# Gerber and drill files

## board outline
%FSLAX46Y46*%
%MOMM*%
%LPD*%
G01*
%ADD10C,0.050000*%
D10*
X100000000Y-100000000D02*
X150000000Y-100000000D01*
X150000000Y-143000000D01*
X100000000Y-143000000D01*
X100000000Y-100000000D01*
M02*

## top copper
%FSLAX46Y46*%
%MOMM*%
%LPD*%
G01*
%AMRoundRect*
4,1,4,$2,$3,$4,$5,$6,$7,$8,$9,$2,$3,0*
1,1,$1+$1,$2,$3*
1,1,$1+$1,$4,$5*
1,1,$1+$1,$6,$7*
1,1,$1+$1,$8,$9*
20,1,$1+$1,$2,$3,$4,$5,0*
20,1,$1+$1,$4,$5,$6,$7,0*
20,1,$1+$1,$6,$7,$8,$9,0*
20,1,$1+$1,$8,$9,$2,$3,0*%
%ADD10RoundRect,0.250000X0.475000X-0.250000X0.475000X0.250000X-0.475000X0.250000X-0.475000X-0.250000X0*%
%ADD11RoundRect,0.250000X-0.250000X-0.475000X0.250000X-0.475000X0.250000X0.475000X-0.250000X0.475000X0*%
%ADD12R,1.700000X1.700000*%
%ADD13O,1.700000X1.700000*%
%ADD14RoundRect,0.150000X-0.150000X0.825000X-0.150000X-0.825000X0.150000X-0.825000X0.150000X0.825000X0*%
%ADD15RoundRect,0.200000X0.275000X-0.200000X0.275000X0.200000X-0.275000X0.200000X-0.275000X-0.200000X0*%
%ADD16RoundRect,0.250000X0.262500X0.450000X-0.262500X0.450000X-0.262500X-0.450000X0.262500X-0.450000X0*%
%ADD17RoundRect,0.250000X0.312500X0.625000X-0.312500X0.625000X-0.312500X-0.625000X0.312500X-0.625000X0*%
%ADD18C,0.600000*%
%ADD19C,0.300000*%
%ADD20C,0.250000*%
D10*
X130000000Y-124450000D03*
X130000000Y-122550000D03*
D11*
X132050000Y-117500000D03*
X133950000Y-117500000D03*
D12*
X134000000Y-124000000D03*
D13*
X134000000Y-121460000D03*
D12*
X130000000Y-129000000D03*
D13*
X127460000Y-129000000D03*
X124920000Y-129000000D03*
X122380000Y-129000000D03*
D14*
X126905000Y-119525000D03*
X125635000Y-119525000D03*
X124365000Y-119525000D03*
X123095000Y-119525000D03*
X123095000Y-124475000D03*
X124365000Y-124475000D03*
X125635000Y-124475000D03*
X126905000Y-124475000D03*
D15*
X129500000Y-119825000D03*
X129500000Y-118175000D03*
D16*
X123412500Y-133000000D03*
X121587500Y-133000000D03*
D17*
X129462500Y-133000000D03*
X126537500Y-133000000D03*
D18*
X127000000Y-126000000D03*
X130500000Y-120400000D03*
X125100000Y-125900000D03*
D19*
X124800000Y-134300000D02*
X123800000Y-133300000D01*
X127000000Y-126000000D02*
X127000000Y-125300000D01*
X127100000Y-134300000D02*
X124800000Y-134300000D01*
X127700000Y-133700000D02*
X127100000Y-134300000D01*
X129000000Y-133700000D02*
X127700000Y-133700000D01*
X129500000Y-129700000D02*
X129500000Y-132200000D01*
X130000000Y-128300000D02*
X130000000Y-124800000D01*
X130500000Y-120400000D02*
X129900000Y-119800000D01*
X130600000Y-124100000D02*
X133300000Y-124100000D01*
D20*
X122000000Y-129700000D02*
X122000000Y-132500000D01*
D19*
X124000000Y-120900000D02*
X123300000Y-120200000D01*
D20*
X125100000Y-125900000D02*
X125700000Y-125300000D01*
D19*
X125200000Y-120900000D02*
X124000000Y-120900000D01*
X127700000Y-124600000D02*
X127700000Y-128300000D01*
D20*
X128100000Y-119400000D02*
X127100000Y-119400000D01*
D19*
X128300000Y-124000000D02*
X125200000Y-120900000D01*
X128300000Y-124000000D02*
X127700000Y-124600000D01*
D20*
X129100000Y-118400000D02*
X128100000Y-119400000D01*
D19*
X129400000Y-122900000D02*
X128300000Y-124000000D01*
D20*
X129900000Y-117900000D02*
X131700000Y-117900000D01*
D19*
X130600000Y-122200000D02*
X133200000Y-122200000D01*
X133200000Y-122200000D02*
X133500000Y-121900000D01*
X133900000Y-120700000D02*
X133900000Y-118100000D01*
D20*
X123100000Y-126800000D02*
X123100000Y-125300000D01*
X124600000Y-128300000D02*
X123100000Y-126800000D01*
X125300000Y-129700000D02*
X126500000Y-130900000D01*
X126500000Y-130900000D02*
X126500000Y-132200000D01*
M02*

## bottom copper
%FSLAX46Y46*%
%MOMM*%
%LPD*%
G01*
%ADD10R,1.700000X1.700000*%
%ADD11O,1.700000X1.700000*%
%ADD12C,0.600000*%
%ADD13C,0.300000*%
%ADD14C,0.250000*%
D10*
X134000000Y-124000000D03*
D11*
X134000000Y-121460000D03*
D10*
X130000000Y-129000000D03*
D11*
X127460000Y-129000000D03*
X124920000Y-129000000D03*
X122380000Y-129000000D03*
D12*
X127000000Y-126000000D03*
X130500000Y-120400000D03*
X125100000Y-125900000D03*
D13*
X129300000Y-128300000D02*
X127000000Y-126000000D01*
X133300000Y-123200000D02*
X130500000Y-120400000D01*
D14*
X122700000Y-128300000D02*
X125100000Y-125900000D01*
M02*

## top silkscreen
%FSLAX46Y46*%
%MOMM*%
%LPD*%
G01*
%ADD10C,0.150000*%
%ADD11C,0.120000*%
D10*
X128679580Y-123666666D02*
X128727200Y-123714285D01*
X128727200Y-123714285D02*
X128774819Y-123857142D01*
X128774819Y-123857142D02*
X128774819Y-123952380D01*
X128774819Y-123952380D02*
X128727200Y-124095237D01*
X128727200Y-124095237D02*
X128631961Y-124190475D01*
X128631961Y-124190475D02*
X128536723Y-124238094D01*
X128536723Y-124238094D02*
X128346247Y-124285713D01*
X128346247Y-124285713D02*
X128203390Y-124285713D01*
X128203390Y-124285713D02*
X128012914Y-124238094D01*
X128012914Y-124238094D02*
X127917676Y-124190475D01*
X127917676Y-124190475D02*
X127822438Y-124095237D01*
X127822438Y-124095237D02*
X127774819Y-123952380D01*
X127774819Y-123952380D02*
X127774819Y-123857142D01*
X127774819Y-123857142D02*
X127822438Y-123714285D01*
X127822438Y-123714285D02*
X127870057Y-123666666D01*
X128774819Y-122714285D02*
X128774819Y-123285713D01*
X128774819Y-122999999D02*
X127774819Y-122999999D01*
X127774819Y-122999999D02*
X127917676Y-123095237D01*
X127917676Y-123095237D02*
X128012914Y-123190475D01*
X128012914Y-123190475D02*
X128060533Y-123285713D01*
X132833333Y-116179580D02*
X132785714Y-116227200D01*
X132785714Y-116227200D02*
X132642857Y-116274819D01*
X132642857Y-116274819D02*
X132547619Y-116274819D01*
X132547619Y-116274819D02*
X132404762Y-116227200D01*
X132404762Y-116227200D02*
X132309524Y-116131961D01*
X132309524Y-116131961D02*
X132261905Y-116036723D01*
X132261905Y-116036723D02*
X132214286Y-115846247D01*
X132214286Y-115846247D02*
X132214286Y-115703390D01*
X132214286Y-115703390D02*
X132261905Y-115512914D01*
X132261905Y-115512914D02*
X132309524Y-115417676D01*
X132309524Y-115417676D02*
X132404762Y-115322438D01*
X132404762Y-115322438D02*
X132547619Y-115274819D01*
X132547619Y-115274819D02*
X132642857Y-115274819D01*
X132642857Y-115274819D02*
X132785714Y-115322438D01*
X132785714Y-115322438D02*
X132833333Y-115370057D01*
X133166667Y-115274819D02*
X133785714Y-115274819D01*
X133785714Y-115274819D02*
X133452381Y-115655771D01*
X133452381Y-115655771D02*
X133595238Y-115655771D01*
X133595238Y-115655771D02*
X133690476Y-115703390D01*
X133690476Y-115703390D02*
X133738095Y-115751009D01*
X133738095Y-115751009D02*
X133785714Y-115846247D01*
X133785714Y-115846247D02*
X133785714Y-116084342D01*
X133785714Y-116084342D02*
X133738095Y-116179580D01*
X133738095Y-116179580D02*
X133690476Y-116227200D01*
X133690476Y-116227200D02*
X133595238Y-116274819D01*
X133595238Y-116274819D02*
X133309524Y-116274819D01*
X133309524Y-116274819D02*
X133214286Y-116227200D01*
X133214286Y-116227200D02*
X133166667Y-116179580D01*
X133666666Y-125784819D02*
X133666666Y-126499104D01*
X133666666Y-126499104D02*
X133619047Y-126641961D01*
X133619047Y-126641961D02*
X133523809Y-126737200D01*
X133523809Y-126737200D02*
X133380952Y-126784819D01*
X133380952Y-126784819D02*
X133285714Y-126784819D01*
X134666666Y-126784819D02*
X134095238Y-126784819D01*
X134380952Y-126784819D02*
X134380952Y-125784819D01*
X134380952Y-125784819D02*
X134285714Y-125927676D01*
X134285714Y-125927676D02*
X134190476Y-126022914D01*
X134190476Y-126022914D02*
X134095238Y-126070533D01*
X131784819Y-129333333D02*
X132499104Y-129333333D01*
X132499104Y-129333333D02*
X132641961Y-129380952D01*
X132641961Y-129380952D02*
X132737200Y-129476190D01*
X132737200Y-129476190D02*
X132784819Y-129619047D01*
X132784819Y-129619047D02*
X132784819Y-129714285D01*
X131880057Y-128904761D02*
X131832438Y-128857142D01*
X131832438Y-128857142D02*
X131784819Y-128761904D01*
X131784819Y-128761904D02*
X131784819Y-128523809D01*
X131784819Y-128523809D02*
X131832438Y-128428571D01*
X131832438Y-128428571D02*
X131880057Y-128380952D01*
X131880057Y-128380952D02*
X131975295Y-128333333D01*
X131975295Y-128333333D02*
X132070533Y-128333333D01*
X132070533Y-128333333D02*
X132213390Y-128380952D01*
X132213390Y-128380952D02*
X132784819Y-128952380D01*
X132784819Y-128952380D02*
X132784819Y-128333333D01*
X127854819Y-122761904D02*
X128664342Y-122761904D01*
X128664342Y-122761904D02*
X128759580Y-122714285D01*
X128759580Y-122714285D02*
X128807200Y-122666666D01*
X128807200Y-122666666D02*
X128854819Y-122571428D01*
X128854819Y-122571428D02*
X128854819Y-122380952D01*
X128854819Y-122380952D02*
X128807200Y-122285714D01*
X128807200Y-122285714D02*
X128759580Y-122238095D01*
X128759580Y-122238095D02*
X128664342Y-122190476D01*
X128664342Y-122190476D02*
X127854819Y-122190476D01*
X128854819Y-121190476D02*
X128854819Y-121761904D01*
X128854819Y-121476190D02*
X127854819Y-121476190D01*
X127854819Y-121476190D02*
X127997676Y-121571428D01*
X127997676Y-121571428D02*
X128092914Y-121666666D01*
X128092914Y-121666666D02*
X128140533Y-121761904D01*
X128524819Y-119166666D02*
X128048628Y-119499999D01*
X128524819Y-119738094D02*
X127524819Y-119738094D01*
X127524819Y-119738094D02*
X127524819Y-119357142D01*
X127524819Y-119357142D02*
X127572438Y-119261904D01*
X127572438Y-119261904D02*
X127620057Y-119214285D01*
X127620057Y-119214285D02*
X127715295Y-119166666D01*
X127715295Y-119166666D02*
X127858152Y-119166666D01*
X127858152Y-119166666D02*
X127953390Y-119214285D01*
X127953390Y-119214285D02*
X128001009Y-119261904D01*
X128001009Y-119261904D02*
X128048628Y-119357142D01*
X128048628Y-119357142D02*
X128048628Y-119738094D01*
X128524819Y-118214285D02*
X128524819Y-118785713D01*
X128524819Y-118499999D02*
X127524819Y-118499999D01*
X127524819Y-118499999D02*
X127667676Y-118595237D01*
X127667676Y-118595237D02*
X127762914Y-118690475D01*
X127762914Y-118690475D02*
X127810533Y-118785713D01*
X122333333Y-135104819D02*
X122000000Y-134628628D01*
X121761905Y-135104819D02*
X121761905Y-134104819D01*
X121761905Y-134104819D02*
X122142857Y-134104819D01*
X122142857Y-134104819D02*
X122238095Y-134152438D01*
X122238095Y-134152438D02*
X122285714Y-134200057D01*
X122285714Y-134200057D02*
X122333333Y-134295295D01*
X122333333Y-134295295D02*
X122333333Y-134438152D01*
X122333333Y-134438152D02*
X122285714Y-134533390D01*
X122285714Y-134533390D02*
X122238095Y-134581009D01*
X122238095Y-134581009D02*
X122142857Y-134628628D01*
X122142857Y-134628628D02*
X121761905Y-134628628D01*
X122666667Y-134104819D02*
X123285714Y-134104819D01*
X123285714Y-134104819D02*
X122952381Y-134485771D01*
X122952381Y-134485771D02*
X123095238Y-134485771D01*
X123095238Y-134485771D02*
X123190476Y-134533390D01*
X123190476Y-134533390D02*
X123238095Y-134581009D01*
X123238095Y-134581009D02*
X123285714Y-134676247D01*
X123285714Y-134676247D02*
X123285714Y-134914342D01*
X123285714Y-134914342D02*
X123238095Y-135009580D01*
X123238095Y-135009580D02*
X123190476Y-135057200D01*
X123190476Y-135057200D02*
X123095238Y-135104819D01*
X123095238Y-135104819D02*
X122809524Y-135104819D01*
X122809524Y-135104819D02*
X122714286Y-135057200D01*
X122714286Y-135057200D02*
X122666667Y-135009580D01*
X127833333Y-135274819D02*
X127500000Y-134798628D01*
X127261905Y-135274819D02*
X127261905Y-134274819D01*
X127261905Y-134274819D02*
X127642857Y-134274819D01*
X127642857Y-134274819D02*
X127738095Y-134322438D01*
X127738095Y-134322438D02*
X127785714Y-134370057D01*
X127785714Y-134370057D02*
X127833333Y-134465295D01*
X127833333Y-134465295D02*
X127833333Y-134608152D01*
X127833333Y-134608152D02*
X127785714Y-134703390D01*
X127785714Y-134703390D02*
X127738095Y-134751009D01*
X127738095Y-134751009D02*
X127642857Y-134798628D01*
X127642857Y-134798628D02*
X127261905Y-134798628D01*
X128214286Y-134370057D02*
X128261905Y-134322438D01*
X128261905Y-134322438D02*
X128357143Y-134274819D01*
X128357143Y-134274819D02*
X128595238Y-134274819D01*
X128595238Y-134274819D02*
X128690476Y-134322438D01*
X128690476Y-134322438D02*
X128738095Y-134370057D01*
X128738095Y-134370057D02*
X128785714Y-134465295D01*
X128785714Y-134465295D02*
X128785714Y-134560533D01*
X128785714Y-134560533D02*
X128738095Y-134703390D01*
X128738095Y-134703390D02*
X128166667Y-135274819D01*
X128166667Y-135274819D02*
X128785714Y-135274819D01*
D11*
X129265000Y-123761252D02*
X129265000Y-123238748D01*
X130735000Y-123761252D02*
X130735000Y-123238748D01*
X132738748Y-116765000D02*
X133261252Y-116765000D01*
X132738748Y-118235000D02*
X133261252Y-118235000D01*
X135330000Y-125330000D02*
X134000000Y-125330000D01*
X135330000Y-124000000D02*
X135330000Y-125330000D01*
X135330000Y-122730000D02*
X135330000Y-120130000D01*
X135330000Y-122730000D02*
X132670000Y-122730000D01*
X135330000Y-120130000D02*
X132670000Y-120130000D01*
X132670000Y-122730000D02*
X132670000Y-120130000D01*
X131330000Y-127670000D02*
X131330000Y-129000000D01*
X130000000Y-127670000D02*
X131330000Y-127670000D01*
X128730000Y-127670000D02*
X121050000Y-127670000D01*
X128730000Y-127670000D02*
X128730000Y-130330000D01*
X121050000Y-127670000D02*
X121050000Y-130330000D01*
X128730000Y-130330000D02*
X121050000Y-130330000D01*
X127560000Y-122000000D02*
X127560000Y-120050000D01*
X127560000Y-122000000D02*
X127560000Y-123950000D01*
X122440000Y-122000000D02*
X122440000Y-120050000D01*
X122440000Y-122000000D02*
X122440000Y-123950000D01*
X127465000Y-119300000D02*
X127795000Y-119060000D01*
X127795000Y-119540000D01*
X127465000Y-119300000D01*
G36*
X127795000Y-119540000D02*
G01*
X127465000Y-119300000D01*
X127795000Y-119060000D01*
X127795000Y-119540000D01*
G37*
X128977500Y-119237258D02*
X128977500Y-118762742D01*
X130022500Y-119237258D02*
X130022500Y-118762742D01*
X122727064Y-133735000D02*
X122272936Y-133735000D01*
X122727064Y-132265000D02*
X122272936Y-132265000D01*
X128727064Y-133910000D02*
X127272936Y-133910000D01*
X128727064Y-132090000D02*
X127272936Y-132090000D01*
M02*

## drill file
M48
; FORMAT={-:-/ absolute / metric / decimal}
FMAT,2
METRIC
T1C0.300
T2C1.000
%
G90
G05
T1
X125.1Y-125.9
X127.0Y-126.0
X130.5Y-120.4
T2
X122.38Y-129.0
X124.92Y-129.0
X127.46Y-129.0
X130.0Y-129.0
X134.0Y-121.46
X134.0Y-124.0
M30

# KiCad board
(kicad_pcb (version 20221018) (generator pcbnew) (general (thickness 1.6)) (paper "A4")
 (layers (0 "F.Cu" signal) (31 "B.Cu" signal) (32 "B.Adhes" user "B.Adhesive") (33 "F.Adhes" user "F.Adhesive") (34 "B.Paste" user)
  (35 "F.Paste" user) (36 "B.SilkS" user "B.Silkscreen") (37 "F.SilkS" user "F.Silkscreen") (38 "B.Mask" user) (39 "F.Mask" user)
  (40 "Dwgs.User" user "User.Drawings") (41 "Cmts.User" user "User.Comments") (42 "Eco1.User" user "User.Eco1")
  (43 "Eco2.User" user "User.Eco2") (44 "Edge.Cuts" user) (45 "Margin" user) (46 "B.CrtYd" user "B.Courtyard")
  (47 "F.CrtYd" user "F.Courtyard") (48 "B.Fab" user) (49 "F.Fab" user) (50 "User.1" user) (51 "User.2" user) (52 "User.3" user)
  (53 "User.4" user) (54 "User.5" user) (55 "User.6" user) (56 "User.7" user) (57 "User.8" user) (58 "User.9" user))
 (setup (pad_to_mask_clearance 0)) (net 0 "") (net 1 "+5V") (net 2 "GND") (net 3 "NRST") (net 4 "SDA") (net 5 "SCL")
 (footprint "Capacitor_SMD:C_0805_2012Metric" (layer "F.Cu") (at 130 123.5 90)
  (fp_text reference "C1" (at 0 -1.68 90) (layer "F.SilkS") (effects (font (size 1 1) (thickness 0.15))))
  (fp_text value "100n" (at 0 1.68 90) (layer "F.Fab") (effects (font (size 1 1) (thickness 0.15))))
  (fp_line (start -0.261252 -0.735) (end 0.261252 -0.735) (stroke (width 0.12) (type solid)) (layer "F.SilkS"))
  (fp_line (start -0.261252 0.735) (end 0.261252 0.735) (stroke (width 0.12) (type solid)) (layer "F.SilkS"))
  (pad "1" smd roundrect (at -0.95 0 90) (size 1 1.45) (layers "F.Cu" "F.Paste" "F.Mask") (roundrect_rratio 0.25) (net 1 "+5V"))
  (pad "2" smd roundrect (at 0.95 0 90) (size 1 1.45) (layers "F.Cu" "F.Paste" "F.Mask") (roundrect_rratio 0.25) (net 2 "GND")))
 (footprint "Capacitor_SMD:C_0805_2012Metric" (layer "F.Cu") (at 133 117.5)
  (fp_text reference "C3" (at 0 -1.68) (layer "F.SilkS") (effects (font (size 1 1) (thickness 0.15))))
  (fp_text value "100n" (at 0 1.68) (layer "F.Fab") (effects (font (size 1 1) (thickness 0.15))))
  (fp_line (start -0.261252 -0.735) (end 0.261252 -0.735) (stroke (width 0.12) (type solid)) (layer "F.SilkS"))
  (fp_line (start -0.261252 0.735) (end 0.261252 0.735) (stroke (width 0.12) (type solid)) (layer "F.SilkS"))
  (pad "1" smd roundrect (at -0.95 0) (size 1 1.45) (layers "F.Cu" "F.Paste" "F.Mask") (roundrect_rratio 0.25) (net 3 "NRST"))
  (pad "2" smd roundrect (at 0.95 0) (size 1 1.45) (layers "F.Cu" "F.Paste" "F.Mask") (roundrect_rratio 0.25) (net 2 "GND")))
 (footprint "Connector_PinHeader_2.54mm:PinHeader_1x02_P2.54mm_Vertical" (layer "F.Cu") (at 134 124 180)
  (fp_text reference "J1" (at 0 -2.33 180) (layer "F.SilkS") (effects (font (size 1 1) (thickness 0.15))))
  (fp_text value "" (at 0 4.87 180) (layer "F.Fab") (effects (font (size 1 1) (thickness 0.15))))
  (fp_line (start -1.33 -1.33) (end 0 -1.33) (stroke (width 0.12) (type solid)) (layer "F.SilkS"))
  (fp_line (start -1.33 0) (end -1.33 -1.33) (stroke (width 0.12) (type solid)) (layer "F.SilkS"))
  (fp_line (start -1.33 1.27) (end -1.33 3.87) (stroke (width 0.12) (type solid)) (layer "F.SilkS"))
  (fp_line (start -1.33 1.27) (end 1.33 1.27) (stroke (width 0.12) (type solid)) (layer "F.SilkS"))
  (fp_line (start -1.33 3.87) (end 1.33 3.87) (stroke (width 0.12) (type solid)) (layer "F.SilkS"))
  (fp_line (start 1.33 1.27) (end 1.33 3.87) (stroke (width 0.12) (type solid)) (layer "F.SilkS"))
  (pad "1" thru_hole rect (at 0 0 180) (size 1.7 1.7) (drill 1) (layers "*.Cu" "*.Mask") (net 1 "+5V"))
  (pad "2" thru_hole oval (at 0 2.54 180) (size 1.7 1.7) (drill 1) (layers "*.Cu" "*.Mask") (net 2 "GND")))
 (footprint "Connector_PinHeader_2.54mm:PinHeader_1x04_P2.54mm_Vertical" (layer "F.Cu") (at 130 129 -90)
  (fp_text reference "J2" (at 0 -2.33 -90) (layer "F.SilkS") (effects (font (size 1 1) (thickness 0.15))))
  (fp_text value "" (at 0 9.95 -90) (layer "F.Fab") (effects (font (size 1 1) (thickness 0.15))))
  (fp_line (start -1.33 -1.33) (end 0 -1.33) (stroke (width 0.12) (type solid)) (layer "F.SilkS"))
  (fp_line (start -1.33 0) (end -1.33 -1.33) (stroke (width 0.12) (type solid)) (layer "F.SilkS"))
  (fp_line (start -1.33 1.27) (end -1.33 8.95) (stroke (width 0.12) (type solid)) (layer "F.SilkS"))
  (fp_line (start -1.33 1.27) (end 1.33 1.27) (stroke (width 0.12) (type solid)) (layer "F.SilkS"))
  (fp_line (start -1.33 8.95) (end 1.33 8.95) (stroke (width 0.12) (type solid)) (layer "F.SilkS"))
  (fp_line (start 1.33 1.27) (end 1.33 8.95) (stroke (width 0.12) (type solid)) (layer "F.SilkS"))
  (pad "1" thru_hole rect (at 0 0 270) (size 1.7 1.7) (drill 1) (layers "*.Cu" "*.Mask") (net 1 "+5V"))
  (pad "2" thru_hole oval (at 0 2.54 270) (size 1.7 1.7) (drill 1) (layers "*.Cu" "*.Mask") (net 2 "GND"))
  (pad "3" thru_hole oval (at 0 5.08 270) (size 1.7 1.7) (drill 1) (layers "*.Cu" "*.Mask") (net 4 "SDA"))
  (pad "4" thru_hole oval (at 0 7.62 270) (size 1.7 1.7) (drill 1) (layers "*.Cu" "*.Mask") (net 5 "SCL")))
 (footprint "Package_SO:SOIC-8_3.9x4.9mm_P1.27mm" (layer "F.Cu") (at 125 122 -90)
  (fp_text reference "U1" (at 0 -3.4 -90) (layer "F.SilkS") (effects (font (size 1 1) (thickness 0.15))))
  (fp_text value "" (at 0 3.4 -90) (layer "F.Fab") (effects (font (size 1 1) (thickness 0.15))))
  (fp_line (start 0 -2.56) (end -1.95 -2.56) (stroke (width 0.12) (type solid)) (layer "F.SilkS"))
  (fp_line (start 0 -2.56) (end 1.95 -2.56) (stroke (width 0.12) (type solid)) (layer "F.SilkS"))
  (fp_line (start 0 2.56) (end -1.95 2.56) (stroke (width 0.12) (type solid)) (layer "F.SilkS"))
  (fp_line (start 0 2.56) (end 1.95 2.56) (stroke (width 0.12) (type solid)) (layer "F.SilkS"))
  (fp_poly
   (pts (xy -2.7 -2.465) (xy -2.94 -2.795) (xy -2.46 -2.795) (xy -2.7 -2.465)) (stroke (width 0.12) (type solid)) (fill solid)
   (layer "F.SilkS"))
  (pad "1" smd roundrect (at -2.475 -1.905 270) (size 1.95 0.6) (layers "F.Cu" "F.Paste" "F.Mask") (roundrect_rratio 0.25) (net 3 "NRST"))
  (pad "2" smd roundrect (at -2.475 -0.635 270) (size 1.95 0.6) (layers "F.Cu" "F.Paste" "F.Mask") (roundrect_rratio 0.25))
  (pad "3" smd roundrect (at -2.475 0.635 270) (size 1.95 0.6) (layers "F.Cu" "F.Paste" "F.Mask") (roundrect_rratio 0.25))
  (pad "4" smd roundrect (at -2.475 1.905 270) (size 1.95 0.6) (layers "F.Cu" "F.Paste" "F.Mask") (roundrect_rratio 0.25) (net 2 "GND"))
  (pad "5" smd roundrect (at 2.475 1.905 270) (size 1.95 0.6) (layers "F.Cu" "F.Paste" "F.Mask") (roundrect_rratio 0.25) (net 4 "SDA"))
  (pad "6" smd roundrect (at 2.475 0.635 270) (size 1.95 0.6) (layers "F.Cu" "F.Paste" "F.Mask") (roundrect_rratio 0.25))
  (pad "7" smd roundrect (at 2.475 -0.635 270) (size 1.95 0.6) (layers "F.Cu" "F.Paste" "F.Mask") (roundrect_rratio 0.25) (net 5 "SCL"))
  (pad "8" smd roundrect (at 2.475 -1.905 270) (size 1.95 0.6) (layers "F.Cu" "F.Paste" "F.Mask") (roundrect_rratio 0.25) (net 1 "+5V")))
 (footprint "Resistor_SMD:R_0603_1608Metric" (layer "F.Cu") (at 129.5 119 90)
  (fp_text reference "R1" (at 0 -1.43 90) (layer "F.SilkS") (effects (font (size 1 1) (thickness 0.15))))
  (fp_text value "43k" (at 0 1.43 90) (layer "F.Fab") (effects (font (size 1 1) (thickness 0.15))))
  (fp_line (start -0.237258 -0.5225) (end 0.237258 -0.5225) (stroke (width 0.12) (type solid)) (layer "F.SilkS"))
  (fp_line (start -0.237258 0.5225) (end 0.237258 0.5225) (stroke (width 0.12) (type solid)) (layer "F.SilkS"))
  (pad "1" smd roundrect (at -0.825 0 90) (size 0.8 0.95) (layers "F.Cu" "F.Paste" "F.Mask") (roundrect_rratio 0.25) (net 1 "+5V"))
  (pad "2" smd roundrect (at 0.825 0 90) (size 0.8 0.95) (layers "F.Cu" "F.Paste" "F.Mask") (roundrect_rratio 0.25) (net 3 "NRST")))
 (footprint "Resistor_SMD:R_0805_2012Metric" (layer "F.Cu") (at 122.5 133 180)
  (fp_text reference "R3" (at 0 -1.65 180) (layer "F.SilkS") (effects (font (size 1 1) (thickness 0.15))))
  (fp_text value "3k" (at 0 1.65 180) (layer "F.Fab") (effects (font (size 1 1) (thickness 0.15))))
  (fp_line (start -0.227064 -0.735) (end 0.227064 -0.735) (stroke (width 0.12) (type solid)) (layer "F.SilkS"))
  (fp_line (start -0.227064 0.735) (end 0.227064 0.735) (stroke (width 0.12) (type solid)) (layer "F.SilkS"))
  (pad "1" smd roundrect (at -0.9125 0 180) (size 1.025 1.4) (layers "F.Cu" "F.Paste" "F.Mask") (roundrect_rratio 0.243902) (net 1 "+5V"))
  (pad "2" smd roundrect (at 0.9125 0 180) (size 1.025 1.4) (layers "F.Cu" "F.Paste" "F.Mask") (roundrect_rratio 0.243902) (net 5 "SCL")))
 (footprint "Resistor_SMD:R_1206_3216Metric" (layer "F.Cu") (at 128 133 180)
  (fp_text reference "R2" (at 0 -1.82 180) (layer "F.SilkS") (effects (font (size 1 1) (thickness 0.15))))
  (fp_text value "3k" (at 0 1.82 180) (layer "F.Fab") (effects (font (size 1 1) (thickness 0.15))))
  (fp_line (start -0.727064 -0.91) (end 0.727064 -0.91) (stroke (width 0.12) (type solid)) (layer "F.SilkS"))
  (fp_line (start -0.727064 0.91) (end 0.727064 0.91) (stroke (width 0.12) (type solid)) (layer "F.SilkS"))
  (pad "1" smd roundrect (at -1.4625 0 180) (size 1.125 1.75) (layers "F.Cu" "F.Paste" "F.Mask") (roundrect_rratio 0.222222) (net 1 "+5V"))
  (pad "2" smd roundrect (at 1.4625 0 180) (size 1.125 1.75) (layers "F.Cu" "F.Paste" "F.Mask") (roundrect_rratio 0.222222) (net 4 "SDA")))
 (gr_rect (start 100 100) (end 150 143) (stroke (width 0.05) (type default)) (fill none) (layer "Edge.Cuts"))
 (segment (start 124.8 134.3) (end 123.8 133.3) (width 0.3) (layer "F.Cu") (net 1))
 (segment (start 127 126) (end 127 125.3) (width 0.3) (layer "F.Cu") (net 1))
 (segment (start 127.1 134.3) (end 124.8 134.3) (width 0.3) (layer "F.Cu") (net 1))
 (segment (start 127.7 133.7) (end 127.1 134.3) (width 0.3) (layer "F.Cu") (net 1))
 (segment (start 129 133.7) (end 127.7 133.7) (width 0.3) (layer "F.Cu") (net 1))
 (segment (start 129.5 129.7) (end 129.5 132.2) (width 0.3) (layer "F.Cu") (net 1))
 (segment (start 130 128.3) (end 130 124.8) (width 0.3) (layer "F.Cu") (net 1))
 (segment (start 130.5 120.4) (end 129.9 119.8) (width 0.3) (layer "F.Cu") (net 1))
 (segment (start 130.6 124.1) (end 133.3 124.1) (width 0.3) (layer "F.Cu") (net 1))
 (via (at 127 126) (size 0.6) (drill 0.3) (layers "F.Cu" "B.Cu") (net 1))
 (via (at 130.5 120.4) (size 0.6) (drill 0.3) (layers "F.Cu" "B.Cu") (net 1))
 (segment (start 122 129.7) (end 122 132.5) (width 0.25) (layer "F.Cu") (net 5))
 (segment (start 124 120.9) (end 123.3 120.2) (width 0.3) (layer "F.Cu") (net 2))
 (segment (start 125.1 125.9) (end 125.7 125.3) (width 0.25) (layer "F.Cu") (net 5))
 (segment (start 125.2 120.9) (end 124 120.9) (width 0.3) (layer "F.Cu") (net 2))
 (segment (start 127.7 124.6) (end 127.7 128.3) (width 0.3) (layer "F.Cu") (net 2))
 (segment (start 128.1 119.4) (end 127.1 119.4) (width 0.25) (layer "F.Cu") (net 3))
 (segment (start 128.3 124) (end 125.2 120.9) (width 0.3) (layer "F.Cu") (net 2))
 (segment (start 128.3 124) (end 127.7 124.6) (width 0.3) (layer "F.Cu") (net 2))
 (segment (start 129.1 118.4) (end 128.1 119.4) (width 0.25) (layer "F.Cu") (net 3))
 (segment (start 129.3 128.3) (end 127 126) (width 0.3) (layer "B.Cu") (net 1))
 (segment (start 129.4 122.9) (end 128.3 124) (width 0.3) (layer "F.Cu") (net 2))
 (segment (start 129.9 117.9) (end 131.7 117.9) (width 0.25) (layer "F.Cu") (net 3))
 (segment (start 130.6 122.2) (end 133.2 122.2) (width 0.3) (layer "F.Cu") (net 2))
 (segment (start 133.2 122.2) (end 133.5 121.9) (width 0.3) (layer "F.Cu") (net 2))
 (segment (start 133.3 123.2) (end 130.5 120.4) (width 0.3) (layer "B.Cu") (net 1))
 (segment (start 133.9 120.7) (end 133.9 118.1) (width 0.3) (layer "F.Cu") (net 2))
 (via (at 125.1 125.9) (size 0.6) (drill 0.3) (layers "F.Cu" "B.Cu") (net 5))
 (segment (start 122.7 128.3) (end 125.1 125.9) (width 0.25) (layer "B.Cu") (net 5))
 (segment (start 123.1 126.8) (end 123.1 125.3) (width 0.25) (layer "F.Cu") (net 4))
 (segment (start 124.6 128.3) (end 123.1 126.8) (width 0.25) (layer "F.Cu") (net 4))
 (segment (start 125.3 129.7) (end 126.5 130.9) (width 0.25) (layer "F.Cu") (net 4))
 (segment (start 126.5 130.9) (end 126.5 132.2) (width 0.25) (layer "F.Cu") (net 4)))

